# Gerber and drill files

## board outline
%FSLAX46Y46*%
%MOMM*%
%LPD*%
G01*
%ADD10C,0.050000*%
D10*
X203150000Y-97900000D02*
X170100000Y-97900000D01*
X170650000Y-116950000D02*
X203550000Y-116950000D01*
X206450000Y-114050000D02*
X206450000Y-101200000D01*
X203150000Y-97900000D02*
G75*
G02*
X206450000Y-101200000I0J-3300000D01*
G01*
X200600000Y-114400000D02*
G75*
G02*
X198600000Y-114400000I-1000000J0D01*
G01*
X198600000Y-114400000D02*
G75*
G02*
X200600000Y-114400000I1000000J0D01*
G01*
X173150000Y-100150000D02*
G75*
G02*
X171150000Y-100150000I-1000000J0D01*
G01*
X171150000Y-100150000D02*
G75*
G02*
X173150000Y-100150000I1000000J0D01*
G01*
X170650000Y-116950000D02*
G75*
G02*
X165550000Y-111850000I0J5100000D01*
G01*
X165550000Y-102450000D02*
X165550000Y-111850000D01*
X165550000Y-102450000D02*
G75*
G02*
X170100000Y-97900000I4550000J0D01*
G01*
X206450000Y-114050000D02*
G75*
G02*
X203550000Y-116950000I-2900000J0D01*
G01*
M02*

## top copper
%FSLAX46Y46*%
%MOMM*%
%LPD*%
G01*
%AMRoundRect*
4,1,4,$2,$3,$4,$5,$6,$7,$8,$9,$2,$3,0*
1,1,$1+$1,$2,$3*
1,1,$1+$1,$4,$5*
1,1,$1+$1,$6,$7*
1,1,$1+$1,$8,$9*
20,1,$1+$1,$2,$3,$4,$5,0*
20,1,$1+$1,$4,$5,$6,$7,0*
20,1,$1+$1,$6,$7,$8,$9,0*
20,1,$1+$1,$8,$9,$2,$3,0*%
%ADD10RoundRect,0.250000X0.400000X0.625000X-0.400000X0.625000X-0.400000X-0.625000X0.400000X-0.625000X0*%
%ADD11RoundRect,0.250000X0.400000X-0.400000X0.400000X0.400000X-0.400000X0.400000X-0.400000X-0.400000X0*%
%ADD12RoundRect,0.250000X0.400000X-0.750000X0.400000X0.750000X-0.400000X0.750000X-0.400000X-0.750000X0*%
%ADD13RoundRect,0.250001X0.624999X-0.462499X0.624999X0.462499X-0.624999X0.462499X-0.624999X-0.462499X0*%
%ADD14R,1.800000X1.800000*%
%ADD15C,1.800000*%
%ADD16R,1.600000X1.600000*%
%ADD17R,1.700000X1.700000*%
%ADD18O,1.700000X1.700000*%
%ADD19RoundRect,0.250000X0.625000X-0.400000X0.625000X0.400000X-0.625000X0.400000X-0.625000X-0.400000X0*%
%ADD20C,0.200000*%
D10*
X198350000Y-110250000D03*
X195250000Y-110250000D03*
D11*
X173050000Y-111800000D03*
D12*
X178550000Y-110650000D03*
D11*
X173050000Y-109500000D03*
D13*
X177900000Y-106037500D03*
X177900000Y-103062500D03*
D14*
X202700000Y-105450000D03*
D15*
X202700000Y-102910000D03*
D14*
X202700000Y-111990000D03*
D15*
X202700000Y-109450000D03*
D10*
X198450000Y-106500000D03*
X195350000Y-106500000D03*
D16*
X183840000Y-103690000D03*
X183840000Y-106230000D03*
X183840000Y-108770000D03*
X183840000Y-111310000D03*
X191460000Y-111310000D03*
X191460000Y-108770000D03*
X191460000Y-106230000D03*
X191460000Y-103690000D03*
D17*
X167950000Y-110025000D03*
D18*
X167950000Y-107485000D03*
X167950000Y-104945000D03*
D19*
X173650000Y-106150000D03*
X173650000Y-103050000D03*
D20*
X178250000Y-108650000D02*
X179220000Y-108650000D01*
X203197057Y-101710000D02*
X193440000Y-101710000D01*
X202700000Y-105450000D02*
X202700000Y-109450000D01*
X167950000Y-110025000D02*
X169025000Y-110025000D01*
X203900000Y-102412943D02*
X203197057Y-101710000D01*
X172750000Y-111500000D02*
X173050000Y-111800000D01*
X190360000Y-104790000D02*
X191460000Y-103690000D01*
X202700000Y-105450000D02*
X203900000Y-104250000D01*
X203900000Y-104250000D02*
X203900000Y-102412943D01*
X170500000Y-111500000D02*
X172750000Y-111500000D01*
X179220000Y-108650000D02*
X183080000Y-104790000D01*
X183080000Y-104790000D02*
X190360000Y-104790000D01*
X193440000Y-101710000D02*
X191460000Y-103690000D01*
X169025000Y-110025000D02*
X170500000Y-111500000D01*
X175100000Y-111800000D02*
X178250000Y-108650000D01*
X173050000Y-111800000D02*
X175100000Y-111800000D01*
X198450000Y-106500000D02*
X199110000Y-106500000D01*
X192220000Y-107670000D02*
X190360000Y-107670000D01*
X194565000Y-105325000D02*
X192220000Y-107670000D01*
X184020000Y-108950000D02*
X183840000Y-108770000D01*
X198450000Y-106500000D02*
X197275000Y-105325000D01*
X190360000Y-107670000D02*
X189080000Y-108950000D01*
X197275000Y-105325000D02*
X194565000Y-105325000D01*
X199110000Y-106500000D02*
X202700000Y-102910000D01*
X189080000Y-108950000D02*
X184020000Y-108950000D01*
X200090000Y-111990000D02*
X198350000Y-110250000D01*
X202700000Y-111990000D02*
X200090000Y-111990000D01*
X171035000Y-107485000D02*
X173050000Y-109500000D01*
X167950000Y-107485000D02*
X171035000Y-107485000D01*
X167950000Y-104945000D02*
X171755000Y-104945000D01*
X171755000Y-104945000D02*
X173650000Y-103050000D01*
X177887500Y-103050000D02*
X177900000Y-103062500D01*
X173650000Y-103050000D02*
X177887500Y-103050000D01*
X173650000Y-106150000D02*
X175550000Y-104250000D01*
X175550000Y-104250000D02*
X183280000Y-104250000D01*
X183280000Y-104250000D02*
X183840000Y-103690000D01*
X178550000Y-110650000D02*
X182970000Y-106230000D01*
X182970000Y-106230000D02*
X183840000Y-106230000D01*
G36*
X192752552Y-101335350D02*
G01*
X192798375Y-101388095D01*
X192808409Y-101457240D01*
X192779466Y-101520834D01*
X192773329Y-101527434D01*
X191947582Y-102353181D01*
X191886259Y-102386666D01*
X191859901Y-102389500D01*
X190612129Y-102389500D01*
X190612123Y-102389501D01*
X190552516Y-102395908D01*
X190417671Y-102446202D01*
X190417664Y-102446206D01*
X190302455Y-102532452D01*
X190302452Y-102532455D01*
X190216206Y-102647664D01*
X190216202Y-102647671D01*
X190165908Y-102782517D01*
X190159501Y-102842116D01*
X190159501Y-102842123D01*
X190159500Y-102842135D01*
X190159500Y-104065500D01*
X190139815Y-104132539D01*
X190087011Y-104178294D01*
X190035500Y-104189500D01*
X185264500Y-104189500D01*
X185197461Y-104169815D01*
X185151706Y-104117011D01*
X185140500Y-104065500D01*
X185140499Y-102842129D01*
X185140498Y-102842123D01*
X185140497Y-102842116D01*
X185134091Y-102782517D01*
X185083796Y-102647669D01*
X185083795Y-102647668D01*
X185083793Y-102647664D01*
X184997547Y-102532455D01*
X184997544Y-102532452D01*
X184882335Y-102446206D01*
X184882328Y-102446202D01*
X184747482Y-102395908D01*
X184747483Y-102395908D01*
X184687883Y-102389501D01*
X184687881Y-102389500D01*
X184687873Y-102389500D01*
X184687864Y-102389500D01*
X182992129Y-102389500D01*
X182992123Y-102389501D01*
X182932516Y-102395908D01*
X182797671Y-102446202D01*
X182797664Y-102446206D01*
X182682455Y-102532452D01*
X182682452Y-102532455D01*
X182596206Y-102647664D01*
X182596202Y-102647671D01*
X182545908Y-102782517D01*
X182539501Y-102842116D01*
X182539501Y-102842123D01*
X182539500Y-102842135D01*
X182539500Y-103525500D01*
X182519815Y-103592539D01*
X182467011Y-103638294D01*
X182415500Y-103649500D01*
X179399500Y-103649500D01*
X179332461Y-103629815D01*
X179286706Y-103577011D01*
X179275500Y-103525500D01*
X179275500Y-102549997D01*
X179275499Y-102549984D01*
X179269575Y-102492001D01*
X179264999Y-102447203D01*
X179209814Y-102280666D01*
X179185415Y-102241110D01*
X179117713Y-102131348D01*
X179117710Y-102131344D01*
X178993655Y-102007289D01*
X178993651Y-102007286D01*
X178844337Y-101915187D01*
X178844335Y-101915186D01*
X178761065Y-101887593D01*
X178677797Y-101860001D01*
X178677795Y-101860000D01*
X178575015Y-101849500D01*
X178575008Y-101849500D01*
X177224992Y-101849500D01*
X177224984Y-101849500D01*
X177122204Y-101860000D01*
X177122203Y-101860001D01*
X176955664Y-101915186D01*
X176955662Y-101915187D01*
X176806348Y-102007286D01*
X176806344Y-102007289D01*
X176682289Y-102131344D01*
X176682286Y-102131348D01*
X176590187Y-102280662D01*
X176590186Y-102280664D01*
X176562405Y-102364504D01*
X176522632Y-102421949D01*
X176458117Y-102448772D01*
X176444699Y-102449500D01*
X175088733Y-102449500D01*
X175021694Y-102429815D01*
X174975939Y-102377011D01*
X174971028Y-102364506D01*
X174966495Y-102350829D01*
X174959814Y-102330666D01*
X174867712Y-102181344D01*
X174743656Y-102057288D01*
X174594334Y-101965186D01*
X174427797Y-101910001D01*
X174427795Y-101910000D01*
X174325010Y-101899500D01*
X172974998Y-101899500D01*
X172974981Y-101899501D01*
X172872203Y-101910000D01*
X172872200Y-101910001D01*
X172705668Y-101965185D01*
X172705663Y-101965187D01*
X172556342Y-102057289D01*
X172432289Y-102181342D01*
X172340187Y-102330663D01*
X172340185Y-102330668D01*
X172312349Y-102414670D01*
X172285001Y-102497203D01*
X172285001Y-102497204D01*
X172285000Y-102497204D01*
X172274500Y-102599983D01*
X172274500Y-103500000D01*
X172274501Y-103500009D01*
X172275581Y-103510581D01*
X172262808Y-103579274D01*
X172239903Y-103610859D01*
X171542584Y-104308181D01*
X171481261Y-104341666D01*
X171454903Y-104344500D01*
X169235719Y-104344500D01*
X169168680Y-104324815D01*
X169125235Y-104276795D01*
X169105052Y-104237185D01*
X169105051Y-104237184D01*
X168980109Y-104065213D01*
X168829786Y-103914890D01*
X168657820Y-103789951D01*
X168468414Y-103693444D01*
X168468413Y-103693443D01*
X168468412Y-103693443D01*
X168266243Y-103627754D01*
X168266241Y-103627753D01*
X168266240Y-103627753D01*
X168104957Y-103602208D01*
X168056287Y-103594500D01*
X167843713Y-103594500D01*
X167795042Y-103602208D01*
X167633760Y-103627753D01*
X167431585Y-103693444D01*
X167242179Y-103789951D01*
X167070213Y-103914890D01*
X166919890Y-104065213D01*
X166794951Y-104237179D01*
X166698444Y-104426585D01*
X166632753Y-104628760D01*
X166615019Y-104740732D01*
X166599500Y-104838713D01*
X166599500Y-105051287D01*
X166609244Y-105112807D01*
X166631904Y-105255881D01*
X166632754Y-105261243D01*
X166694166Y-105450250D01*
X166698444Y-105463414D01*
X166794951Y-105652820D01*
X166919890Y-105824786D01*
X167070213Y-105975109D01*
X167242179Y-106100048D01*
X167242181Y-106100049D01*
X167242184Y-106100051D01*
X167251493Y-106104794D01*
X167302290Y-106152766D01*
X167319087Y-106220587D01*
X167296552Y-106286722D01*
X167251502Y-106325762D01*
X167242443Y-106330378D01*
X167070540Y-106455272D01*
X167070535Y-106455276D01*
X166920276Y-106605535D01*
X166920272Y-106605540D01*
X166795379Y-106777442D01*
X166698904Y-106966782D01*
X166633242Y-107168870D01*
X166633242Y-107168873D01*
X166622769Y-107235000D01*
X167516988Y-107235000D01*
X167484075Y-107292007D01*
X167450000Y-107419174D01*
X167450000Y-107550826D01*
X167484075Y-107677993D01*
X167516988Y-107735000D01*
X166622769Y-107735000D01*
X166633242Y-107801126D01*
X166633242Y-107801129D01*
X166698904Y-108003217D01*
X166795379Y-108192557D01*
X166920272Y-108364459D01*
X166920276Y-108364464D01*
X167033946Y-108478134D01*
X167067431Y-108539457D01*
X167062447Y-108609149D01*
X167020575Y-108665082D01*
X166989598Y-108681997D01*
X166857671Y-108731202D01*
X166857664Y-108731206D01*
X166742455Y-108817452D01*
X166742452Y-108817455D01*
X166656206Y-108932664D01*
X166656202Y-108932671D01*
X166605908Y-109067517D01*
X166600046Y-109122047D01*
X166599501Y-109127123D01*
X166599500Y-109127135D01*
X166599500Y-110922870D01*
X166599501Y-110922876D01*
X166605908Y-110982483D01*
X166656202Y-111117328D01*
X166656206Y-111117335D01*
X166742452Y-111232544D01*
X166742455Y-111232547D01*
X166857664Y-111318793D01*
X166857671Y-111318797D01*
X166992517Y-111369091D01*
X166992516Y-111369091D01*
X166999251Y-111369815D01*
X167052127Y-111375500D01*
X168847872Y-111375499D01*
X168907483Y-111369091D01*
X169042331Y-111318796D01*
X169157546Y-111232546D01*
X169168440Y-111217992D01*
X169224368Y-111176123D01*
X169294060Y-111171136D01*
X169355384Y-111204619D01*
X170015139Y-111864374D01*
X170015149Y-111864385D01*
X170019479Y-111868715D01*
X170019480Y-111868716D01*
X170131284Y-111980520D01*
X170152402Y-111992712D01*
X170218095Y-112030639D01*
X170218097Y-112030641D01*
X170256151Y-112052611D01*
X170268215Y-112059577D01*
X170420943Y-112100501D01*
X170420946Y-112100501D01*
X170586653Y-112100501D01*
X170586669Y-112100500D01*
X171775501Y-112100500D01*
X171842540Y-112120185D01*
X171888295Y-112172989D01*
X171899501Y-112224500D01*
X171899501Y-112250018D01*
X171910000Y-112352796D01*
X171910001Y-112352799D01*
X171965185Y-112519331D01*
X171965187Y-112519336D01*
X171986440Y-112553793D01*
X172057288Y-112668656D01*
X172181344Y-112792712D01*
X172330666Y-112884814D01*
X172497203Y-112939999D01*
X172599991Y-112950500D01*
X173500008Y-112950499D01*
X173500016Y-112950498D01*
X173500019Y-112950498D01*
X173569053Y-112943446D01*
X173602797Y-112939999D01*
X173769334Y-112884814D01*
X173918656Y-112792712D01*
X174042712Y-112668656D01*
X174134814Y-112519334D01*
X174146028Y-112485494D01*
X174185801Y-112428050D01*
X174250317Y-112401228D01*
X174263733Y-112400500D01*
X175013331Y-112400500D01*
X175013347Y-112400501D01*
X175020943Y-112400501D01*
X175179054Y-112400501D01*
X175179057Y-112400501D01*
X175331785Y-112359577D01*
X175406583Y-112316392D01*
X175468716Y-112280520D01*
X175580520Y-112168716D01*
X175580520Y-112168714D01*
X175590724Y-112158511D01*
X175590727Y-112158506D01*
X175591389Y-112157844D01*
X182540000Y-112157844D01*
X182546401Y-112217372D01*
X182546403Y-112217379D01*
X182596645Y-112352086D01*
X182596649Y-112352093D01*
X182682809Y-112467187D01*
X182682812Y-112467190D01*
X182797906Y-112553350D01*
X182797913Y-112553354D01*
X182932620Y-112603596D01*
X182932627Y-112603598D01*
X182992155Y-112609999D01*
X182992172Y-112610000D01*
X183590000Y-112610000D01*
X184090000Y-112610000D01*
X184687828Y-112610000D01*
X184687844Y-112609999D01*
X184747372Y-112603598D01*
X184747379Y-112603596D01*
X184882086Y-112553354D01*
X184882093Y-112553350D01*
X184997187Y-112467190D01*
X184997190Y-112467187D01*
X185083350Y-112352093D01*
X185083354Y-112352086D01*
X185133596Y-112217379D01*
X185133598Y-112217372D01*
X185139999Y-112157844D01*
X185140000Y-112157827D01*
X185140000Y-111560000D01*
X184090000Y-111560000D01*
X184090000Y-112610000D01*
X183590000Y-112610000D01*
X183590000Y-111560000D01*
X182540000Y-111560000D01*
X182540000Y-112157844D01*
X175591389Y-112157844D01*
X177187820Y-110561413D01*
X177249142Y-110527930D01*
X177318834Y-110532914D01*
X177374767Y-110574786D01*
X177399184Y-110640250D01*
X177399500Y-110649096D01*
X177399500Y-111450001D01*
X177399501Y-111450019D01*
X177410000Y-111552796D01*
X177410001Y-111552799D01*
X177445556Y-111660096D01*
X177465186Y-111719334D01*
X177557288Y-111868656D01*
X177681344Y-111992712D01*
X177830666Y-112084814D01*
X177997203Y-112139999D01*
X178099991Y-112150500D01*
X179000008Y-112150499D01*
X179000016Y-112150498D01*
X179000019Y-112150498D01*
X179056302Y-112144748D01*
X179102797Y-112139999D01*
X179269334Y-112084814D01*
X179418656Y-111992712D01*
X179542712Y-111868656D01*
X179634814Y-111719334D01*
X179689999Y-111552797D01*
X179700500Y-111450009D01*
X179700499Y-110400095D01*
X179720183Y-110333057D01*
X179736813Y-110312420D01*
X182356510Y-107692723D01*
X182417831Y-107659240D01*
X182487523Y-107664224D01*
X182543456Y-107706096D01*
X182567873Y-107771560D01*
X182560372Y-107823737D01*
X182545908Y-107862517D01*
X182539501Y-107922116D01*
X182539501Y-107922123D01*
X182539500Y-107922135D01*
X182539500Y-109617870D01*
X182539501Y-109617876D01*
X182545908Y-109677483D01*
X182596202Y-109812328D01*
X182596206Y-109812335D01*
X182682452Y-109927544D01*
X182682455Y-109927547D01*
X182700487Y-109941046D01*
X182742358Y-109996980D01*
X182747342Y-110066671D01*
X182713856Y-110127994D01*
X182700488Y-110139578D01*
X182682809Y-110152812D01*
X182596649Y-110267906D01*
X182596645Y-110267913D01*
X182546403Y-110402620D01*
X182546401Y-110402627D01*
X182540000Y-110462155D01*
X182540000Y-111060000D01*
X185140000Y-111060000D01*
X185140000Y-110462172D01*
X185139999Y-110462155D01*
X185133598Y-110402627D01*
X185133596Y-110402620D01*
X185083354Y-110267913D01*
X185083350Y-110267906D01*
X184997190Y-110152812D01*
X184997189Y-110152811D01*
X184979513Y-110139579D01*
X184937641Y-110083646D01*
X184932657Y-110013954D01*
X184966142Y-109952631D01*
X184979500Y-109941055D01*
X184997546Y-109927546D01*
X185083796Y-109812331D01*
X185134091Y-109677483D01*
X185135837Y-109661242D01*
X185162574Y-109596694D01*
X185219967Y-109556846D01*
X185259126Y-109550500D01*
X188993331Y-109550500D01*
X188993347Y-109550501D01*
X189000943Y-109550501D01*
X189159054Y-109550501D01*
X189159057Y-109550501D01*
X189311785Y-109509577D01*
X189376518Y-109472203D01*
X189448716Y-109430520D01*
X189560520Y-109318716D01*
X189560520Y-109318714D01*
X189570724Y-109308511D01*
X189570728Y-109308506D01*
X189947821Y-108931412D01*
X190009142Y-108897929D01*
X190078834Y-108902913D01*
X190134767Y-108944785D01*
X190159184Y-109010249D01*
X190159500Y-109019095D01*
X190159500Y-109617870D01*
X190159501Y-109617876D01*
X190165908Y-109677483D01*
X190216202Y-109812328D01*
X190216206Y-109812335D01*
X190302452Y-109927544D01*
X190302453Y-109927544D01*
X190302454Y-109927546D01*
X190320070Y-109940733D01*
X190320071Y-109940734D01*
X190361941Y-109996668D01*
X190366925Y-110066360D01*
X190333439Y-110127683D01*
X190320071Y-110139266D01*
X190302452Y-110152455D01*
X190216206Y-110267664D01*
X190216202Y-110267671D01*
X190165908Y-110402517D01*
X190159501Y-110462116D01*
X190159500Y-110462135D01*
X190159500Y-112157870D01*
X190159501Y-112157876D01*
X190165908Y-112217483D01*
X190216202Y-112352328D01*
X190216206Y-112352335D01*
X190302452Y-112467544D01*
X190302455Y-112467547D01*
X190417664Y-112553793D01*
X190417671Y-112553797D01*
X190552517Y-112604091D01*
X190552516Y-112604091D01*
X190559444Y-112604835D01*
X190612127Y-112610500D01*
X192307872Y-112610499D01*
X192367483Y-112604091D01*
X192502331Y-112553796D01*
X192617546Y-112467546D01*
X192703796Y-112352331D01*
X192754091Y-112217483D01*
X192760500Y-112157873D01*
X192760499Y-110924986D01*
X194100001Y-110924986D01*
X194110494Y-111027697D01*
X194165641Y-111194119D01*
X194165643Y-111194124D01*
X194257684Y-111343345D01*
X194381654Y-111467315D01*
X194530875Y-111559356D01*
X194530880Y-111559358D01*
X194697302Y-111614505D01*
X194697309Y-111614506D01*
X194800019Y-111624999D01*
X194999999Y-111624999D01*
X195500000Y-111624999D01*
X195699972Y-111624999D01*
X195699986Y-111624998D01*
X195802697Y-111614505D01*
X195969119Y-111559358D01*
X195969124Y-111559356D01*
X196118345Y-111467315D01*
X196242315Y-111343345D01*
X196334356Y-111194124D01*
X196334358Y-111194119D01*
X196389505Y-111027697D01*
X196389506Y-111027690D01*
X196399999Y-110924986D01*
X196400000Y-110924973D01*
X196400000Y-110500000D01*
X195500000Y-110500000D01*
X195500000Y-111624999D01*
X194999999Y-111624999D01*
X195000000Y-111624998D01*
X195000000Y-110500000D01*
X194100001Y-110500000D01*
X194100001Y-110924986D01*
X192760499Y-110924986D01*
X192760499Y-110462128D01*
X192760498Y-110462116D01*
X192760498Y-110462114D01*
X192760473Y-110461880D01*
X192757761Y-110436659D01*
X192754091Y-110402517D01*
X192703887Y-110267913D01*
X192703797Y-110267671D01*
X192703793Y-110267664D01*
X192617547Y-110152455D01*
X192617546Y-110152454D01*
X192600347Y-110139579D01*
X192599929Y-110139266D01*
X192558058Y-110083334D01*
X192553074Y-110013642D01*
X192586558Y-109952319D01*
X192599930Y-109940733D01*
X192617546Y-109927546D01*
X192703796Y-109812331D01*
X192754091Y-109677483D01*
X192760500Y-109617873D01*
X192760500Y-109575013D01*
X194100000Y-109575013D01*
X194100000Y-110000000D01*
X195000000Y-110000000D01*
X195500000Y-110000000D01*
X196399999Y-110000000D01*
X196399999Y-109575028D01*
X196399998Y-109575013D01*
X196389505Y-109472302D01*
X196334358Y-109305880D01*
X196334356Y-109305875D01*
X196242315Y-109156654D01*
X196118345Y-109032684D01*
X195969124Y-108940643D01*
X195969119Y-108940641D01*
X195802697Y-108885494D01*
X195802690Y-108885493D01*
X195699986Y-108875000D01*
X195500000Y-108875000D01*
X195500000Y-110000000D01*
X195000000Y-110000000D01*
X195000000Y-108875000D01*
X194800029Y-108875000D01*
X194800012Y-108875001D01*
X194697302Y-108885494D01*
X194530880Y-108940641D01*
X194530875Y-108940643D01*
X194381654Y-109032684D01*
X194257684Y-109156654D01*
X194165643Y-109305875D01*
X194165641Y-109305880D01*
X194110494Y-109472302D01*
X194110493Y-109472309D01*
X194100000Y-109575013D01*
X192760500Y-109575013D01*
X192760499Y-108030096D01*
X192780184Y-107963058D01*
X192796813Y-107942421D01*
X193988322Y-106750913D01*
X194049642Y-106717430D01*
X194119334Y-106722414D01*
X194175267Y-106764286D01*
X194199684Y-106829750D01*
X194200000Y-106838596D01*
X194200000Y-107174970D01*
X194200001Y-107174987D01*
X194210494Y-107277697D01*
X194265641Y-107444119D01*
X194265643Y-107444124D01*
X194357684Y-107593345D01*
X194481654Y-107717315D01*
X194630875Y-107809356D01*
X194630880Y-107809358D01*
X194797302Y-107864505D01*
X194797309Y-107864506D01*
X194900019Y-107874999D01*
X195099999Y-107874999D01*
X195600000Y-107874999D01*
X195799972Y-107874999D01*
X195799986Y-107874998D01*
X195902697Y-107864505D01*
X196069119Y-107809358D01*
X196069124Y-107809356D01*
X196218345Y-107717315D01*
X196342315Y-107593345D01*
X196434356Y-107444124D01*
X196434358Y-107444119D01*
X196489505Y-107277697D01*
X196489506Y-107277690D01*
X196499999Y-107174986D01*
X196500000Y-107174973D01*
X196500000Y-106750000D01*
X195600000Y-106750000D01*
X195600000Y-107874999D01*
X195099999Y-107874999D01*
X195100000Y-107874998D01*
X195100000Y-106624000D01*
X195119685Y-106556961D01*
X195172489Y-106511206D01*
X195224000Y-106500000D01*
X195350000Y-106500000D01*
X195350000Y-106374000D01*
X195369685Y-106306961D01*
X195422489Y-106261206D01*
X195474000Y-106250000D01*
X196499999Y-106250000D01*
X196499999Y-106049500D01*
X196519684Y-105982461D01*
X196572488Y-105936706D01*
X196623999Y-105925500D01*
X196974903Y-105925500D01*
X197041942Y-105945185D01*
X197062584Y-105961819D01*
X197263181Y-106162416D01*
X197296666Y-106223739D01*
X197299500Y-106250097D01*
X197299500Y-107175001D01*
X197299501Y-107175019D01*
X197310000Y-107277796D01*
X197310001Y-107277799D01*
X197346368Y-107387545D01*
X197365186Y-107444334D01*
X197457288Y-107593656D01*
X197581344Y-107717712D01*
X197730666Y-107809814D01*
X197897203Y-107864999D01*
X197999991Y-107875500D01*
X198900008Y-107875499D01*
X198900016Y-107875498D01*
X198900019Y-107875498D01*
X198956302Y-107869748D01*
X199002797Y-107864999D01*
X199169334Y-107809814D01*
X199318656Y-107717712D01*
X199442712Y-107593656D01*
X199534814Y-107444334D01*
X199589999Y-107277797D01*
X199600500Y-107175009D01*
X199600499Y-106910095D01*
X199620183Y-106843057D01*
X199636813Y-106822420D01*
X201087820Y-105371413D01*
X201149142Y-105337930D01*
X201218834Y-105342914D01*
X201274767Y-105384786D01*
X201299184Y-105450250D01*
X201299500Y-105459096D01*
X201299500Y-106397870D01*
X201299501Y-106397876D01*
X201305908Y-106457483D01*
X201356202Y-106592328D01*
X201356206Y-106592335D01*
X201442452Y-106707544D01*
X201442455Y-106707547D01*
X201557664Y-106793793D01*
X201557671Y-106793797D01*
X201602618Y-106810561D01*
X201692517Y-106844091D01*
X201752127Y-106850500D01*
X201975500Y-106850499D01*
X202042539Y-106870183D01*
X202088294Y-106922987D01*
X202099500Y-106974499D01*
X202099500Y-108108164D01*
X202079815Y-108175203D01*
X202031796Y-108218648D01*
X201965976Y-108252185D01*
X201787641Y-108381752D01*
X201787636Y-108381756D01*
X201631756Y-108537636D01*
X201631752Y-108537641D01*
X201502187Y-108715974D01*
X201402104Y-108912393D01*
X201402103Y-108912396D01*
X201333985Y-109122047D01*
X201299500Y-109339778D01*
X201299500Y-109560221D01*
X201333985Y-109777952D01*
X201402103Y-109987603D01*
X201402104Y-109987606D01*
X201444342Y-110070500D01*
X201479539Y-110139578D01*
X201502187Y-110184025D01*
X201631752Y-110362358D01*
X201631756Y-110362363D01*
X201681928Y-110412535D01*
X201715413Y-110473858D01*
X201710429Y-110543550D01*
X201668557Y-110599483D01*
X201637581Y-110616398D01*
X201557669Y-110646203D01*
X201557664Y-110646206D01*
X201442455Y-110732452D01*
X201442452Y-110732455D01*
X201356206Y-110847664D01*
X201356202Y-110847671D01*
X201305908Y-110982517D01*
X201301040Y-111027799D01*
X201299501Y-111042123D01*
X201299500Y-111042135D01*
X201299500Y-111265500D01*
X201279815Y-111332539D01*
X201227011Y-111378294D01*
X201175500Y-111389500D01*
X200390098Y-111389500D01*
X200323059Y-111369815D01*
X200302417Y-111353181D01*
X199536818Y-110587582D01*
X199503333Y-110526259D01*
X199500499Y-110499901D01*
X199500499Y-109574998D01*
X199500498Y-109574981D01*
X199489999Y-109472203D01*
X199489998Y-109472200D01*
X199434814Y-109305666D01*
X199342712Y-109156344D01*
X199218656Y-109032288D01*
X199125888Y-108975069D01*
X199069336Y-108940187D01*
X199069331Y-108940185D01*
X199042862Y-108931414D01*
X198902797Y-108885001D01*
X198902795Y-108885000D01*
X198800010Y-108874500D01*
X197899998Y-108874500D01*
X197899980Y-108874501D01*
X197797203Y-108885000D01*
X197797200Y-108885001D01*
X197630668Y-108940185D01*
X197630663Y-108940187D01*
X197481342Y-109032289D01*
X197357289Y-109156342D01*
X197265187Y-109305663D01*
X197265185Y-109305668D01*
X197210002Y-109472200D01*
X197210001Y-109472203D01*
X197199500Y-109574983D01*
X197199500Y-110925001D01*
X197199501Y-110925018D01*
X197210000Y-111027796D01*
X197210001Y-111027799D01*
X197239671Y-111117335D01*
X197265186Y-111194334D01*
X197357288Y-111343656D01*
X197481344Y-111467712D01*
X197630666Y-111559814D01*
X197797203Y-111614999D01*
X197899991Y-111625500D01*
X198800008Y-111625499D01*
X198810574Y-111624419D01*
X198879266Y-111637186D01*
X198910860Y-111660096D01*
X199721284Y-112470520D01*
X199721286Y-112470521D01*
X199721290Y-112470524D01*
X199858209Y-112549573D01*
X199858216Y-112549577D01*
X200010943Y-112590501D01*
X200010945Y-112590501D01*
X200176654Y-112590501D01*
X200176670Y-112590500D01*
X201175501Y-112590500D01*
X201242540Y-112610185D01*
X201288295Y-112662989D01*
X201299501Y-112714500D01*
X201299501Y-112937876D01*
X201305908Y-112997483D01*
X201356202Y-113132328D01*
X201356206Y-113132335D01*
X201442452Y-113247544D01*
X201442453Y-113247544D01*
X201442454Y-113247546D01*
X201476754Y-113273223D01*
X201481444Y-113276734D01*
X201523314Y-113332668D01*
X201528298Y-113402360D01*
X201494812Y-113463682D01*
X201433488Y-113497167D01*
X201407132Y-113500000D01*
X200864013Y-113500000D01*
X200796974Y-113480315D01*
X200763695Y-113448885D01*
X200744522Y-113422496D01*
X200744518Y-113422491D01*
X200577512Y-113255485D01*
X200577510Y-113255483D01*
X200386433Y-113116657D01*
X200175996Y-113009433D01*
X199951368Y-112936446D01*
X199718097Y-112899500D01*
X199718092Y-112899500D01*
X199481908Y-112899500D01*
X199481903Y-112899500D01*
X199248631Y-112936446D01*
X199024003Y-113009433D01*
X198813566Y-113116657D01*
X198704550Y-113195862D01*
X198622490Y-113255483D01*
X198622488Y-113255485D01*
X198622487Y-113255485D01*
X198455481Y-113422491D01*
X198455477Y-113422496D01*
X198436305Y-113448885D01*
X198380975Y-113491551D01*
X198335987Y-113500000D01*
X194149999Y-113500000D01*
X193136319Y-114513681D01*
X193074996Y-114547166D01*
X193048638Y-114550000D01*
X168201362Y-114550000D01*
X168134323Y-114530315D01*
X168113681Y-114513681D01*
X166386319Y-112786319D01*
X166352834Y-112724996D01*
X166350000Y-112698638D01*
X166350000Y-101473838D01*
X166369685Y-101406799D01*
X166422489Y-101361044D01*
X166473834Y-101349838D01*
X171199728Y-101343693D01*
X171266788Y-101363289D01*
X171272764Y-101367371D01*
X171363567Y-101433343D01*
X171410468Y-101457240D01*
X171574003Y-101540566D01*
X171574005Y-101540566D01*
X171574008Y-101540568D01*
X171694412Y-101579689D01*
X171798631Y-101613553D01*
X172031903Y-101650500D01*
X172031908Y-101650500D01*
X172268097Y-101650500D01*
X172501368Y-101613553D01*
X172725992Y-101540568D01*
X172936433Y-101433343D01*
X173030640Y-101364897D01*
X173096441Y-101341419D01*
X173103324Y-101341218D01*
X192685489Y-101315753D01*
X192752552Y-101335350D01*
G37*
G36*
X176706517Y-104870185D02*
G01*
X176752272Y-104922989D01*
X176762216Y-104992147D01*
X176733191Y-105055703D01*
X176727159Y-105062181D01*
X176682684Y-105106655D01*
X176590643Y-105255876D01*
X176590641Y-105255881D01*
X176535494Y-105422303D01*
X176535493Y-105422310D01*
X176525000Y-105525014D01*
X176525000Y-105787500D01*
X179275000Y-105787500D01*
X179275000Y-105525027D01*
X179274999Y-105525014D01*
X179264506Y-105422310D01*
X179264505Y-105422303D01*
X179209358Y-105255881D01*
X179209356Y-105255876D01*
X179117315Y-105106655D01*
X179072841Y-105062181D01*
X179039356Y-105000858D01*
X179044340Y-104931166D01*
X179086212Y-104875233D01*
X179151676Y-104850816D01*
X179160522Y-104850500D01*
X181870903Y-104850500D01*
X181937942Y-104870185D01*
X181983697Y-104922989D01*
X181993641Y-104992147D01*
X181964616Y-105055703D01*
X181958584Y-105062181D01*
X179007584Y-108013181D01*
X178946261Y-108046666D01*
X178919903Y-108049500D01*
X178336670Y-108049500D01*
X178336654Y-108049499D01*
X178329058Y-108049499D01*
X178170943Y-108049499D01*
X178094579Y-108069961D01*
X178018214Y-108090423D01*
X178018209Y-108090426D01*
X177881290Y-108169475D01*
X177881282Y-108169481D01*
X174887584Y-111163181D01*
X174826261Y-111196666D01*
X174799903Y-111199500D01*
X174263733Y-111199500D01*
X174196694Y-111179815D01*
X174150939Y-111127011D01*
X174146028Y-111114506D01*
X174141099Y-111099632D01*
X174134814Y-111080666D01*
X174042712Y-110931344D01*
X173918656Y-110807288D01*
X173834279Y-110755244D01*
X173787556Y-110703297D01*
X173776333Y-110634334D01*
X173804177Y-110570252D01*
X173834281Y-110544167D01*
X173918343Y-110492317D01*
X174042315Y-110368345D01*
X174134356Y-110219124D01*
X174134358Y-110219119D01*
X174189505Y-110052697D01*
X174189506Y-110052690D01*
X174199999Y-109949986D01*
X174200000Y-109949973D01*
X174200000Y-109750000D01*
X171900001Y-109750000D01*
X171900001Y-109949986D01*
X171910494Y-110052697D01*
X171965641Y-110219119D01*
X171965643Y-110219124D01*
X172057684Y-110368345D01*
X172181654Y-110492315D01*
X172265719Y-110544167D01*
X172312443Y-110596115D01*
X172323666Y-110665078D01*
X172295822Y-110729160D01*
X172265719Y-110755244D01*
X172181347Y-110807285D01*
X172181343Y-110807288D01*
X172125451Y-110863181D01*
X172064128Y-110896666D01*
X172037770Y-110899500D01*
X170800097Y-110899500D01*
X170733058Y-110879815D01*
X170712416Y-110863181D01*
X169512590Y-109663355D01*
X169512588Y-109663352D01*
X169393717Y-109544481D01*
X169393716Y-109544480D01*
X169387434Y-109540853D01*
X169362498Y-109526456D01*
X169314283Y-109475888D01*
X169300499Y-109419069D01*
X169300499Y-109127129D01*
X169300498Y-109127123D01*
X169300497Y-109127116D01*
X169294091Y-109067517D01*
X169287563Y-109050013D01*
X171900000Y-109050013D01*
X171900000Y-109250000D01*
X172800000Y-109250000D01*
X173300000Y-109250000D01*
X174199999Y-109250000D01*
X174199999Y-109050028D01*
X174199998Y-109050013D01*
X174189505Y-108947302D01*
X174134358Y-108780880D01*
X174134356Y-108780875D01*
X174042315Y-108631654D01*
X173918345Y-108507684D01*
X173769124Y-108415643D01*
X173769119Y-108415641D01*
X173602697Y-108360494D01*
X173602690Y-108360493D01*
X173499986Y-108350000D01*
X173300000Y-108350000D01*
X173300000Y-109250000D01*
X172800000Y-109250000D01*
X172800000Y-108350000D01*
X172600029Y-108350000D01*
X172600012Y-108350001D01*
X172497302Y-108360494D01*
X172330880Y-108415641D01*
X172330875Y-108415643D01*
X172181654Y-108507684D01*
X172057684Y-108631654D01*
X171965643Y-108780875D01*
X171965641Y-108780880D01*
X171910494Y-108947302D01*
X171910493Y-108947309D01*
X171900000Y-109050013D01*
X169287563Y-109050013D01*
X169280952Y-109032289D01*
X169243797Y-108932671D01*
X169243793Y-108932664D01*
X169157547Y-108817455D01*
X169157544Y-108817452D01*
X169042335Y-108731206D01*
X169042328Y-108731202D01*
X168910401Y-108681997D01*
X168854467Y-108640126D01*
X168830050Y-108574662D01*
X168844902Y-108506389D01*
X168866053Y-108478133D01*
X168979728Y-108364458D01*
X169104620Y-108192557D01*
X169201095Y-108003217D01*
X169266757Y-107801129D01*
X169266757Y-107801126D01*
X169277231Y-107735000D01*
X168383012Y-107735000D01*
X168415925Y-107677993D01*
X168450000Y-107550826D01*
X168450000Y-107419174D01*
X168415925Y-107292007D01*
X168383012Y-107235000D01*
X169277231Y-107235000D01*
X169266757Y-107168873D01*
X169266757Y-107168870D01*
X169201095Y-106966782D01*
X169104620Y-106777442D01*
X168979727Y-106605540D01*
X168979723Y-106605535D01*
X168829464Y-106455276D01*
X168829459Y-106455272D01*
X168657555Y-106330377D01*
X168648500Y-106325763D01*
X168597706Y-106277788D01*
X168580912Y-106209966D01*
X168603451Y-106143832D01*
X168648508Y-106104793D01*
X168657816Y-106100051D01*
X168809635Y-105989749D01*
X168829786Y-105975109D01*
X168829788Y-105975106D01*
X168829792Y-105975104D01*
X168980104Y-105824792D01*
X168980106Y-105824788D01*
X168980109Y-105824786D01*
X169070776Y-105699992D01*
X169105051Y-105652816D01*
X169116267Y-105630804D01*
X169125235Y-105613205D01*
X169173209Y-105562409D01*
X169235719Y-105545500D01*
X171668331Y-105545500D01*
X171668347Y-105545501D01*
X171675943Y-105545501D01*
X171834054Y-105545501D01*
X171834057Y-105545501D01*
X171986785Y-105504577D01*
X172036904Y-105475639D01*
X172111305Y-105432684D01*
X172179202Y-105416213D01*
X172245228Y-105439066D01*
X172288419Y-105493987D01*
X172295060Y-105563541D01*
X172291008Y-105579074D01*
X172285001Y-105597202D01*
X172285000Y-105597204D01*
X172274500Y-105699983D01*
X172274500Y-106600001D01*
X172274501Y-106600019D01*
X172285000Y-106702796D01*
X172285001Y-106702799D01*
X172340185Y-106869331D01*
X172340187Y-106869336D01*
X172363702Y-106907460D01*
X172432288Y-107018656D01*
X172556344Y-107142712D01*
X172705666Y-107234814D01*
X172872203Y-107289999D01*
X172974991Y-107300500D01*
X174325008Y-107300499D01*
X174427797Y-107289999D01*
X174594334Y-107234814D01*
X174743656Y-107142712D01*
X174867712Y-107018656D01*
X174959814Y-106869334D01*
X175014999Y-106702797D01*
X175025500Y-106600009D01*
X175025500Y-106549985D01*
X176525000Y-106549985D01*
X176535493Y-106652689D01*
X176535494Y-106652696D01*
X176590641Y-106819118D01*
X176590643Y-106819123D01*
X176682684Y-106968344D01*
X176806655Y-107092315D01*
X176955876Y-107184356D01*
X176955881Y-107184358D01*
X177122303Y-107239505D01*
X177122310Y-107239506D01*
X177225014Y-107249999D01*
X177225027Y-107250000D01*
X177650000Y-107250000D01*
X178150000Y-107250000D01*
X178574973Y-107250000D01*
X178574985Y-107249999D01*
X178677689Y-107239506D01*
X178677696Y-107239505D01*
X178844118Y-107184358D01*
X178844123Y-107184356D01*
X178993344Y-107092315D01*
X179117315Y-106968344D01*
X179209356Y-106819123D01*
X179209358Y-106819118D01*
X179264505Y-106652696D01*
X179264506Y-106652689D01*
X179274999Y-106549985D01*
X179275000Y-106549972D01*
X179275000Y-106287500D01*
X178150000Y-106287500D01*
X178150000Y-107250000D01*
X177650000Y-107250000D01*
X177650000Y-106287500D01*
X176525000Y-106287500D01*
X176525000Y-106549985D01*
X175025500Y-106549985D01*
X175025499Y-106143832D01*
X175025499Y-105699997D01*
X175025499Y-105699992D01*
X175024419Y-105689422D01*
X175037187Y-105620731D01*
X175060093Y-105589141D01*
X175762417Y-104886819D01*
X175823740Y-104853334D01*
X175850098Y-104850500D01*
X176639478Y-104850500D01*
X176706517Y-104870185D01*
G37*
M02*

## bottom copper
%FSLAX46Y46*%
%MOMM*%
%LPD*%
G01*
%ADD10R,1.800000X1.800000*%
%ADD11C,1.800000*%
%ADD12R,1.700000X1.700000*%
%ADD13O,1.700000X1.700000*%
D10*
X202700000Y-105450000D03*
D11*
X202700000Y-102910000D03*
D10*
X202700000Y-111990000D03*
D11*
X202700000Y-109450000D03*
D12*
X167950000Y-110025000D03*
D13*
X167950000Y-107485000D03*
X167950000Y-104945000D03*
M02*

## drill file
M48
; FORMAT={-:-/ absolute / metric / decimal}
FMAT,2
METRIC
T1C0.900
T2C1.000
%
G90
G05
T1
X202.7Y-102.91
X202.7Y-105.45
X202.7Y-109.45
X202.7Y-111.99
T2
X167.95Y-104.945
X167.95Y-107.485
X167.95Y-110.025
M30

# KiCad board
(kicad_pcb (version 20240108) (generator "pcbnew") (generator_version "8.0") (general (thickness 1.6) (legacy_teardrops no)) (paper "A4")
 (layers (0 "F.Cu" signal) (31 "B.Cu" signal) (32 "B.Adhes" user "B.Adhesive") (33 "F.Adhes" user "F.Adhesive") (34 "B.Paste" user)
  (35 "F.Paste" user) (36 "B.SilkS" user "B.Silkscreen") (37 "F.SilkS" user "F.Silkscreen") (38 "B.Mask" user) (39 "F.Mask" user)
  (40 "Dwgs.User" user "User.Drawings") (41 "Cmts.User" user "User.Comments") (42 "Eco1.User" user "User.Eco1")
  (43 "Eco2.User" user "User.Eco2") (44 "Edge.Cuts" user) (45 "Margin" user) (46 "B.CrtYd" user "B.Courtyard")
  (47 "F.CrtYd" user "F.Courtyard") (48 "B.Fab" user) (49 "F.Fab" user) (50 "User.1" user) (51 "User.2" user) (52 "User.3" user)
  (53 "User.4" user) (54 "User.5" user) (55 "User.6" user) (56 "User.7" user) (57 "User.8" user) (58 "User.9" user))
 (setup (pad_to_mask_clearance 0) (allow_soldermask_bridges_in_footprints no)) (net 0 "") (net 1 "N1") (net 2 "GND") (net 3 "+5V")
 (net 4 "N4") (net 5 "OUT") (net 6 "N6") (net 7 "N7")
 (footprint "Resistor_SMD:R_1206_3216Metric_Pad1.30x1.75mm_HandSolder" (layer "F.Cu") (at 196.8 110.25 180)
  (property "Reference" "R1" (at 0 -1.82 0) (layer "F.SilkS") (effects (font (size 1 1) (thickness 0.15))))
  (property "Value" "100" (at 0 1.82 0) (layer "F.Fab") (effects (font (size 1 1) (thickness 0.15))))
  (pad "1" smd roundrect (at -1.55 0 180) (size 1.3 1.75) (layers "F.Cu" "F.Paste" "F.Mask") (roundrect_rratio 0.192308) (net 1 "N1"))
  (pad "2" smd roundrect (at 1.55 0 180) (size 1.3 1.75) (layers "F.Cu" "F.Paste" "F.Mask") (roundrect_rratio 0.192308) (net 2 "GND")))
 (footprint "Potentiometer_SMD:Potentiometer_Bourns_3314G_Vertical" (layer "F.Cu") (at 175.8 110.65 90)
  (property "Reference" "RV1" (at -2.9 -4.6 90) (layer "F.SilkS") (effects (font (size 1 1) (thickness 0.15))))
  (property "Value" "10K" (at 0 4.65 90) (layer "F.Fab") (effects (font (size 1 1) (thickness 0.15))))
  (pad "1" smd roundrect (at -1.15 -2.75 90) (size 1.3 1.3) (layers "F.Cu" "F.Paste" "F.Mask") (roundrect_rratio 0.1923076923) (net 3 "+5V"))
  (pad "2" smd roundrect (at 0 2.75 90) (size 2 1.3) (layers "F.Cu" "F.Paste" "F.Mask") (roundrect_rratio 0.1923076923) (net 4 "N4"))
  (pad "3" smd roundrect (at 1.15 -2.75 90) (size 1.3 1.3) (layers "F.Cu" "F.Paste" "F.Mask") (roundrect_rratio 0.1923076923) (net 2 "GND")))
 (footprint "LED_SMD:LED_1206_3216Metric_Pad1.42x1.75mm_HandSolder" (layer "F.Cu") (at 177.9 104.55 90)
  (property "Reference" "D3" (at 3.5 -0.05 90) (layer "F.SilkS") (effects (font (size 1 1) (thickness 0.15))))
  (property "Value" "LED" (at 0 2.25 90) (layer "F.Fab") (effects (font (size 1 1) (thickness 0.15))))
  (pad "1" smd roundrect (at -1.4875 0 90) (size 1.425 1.75) (layers "F.Cu" "F.Paste" "F.Mask") (roundrect_rratio 0.175439) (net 2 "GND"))
  (pad "2" smd roundrect (at 1.4875 0 90) (size 1.425 1.75) (layers "F.Cu" "F.Paste" "F.Mask") (roundrect_rratio 0.175439) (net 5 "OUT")))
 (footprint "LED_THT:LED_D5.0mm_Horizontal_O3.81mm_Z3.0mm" (layer "F.Cu") (at 202.7 105.45 90)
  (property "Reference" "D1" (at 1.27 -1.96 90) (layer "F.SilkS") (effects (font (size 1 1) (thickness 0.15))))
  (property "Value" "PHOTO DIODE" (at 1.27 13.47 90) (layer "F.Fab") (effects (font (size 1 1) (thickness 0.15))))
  (pad "1" thru_hole rect (at 0 0 90) (size 1.8 1.8) (drill 0.9) (layers "*.Cu" "*.Mask") (remove_unused_layers no) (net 3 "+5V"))
  (pad "2" thru_hole circle (at 2.54 0 90) (size 1.8 1.8) (drill 0.9) (layers "*.Cu" "*.Mask") (remove_unused_layers no) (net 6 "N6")))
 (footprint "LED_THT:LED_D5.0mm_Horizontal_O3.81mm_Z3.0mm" (layer "F.Cu") (at 202.7 111.99 90)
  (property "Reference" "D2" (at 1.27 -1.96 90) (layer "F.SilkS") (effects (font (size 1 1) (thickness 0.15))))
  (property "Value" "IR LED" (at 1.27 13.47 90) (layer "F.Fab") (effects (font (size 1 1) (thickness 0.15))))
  (pad "1" thru_hole rect (at 0 0 90) (size 1.8 1.8) (drill 0.9) (layers "*.Cu" "*.Mask") (remove_unused_layers no) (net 1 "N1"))
  (pad "2" thru_hole circle (at 2.54 0 90) (size 1.8 1.8) (drill 0.9) (layers "*.Cu" "*.Mask") (remove_unused_layers no) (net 3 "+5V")))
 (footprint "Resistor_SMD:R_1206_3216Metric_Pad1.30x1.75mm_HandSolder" (layer "F.Cu") (at 196.9 106.5 180)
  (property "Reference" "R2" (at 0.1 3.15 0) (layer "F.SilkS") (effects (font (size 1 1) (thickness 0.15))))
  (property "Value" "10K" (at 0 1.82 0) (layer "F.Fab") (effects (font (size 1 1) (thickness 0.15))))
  (pad "1" smd roundrect (at -1.55 0 180) (size 1.3 1.75) (layers "F.Cu" "F.Paste" "F.Mask") (roundrect_rratio 0.192308) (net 6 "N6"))
  (pad "2" smd roundrect (at 1.55 0 180) (size 1.3 1.75) (layers "F.Cu" "F.Paste" "F.Mask") (roundrect_rratio 0.192308) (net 2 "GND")))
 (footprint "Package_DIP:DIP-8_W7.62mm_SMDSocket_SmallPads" (layer "F.Cu") (at 187.65 107.5)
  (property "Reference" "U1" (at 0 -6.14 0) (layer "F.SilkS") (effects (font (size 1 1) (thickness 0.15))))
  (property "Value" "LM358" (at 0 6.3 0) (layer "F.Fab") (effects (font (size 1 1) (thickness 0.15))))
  (pad "1" smd rect (at -3.81 -3.81) (size 1.6 1.6) (layers "F.Cu" "F.Paste" "F.Mask") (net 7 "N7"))
  (pad "2" smd rect (at -3.81 -1.27) (size 1.6 1.6) (layers "F.Cu" "F.Paste" "F.Mask") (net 4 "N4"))
  (pad "3" smd rect (at -3.81 1.27) (size 1.6 1.6) (layers "F.Cu" "F.Paste" "F.Mask") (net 6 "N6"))
  (pad "4" smd rect (at -3.81 3.81) (size 1.6 1.6) (layers "F.Cu" "F.Paste" "F.Mask") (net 2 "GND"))
  (pad "5" smd rect (at 3.81 3.81) (size 1.6 1.6) (layers "F.Cu" "F.Paste" "F.Mask"))
  (pad "6" smd rect (at 3.81 1.27) (size 1.6 1.6) (layers "F.Cu" "F.Paste" "F.Mask"))
  (pad "7" smd rect (at 3.81 -1.27) (size 1.6 1.6) (layers "F.Cu" "F.Paste" "F.Mask"))
  (pad "8" smd rect (at 3.81 -3.81) (size 1.6 1.6) (layers "F.Cu" "F.Paste" "F.Mask") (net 3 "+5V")))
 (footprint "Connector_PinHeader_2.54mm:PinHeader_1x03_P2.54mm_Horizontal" (layer "F.Cu") (at 167.95 110.025 180)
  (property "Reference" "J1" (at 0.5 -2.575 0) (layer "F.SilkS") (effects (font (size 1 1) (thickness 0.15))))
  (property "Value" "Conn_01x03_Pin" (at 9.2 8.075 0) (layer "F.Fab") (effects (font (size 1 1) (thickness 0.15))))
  (pad "1" thru_hole rect (at 0 0 180) (size 1.7 1.7) (drill 1) (layers "*.Cu" "*.Mask") (remove_unused_layers no) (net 3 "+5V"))
  (pad "2" thru_hole oval (at 0 2.54 180) (size 1.7 1.7) (drill 1) (layers "*.Cu" "*.Mask") (remove_unused_layers no) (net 2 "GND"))
  (pad "3" thru_hole oval (at 0 5.08 180) (size 1.7 1.7) (drill 1) (layers "*.Cu" "*.Mask") (remove_unused_layers no) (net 5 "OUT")))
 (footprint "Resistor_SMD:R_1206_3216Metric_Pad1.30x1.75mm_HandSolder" (layer "F.Cu") (at 173.65 104.6 90)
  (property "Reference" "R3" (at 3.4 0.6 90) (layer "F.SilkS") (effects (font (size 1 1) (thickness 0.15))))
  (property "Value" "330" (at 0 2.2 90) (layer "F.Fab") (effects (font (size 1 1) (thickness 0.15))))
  (pad "1" smd roundrect (at -1.55 0 90) (size 1.3 1.75) (layers "F.Cu" "F.Paste" "F.Mask") (roundrect_rratio 0.192308) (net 7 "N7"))
  (pad "2" smd roundrect (at 1.55 0 90) (size 1.3 1.75) (layers "F.Cu" "F.Paste" "F.Mask") (roundrect_rratio 0.192308) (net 5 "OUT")))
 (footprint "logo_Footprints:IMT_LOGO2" (layer "B.Cu") (at 187.825 102.12 180)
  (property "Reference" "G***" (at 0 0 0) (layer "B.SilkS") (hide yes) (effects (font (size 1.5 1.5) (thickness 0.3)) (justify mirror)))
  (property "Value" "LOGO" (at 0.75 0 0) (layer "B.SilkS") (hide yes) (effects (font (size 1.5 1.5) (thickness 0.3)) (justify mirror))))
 (gr_line (start 203.15 97.9) (end 170.1 97.9) (stroke (width 0.05) (type default)) (layer "Edge.Cuts"))
 (gr_line (start 170.65 116.95) (end 203.55 116.95) (stroke (width 0.05) (type default)) (layer "Edge.Cuts"))
 (gr_line (start 206.45 114.05) (end 206.45 101.2) (stroke (width 0.05) (type default)) (layer "Edge.Cuts"))
 (gr_arc (start 203.15 97.9) (mid 205.483452 98.866548) (end 206.45 101.2) (stroke (width 0.05) (type default)) (layer "Edge.Cuts"))
 (gr_circle (center 199.6 114.4) (end 199.6 113.4) (stroke (width 0.05) (type default)) (fill none) (layer "Edge.Cuts"))
 (gr_circle (center 172.15 100.15) (end 172.15 99.15) (stroke (width 0.05) (type default)) (fill none) (layer "Edge.Cuts"))
 (gr_arc (start 170.65 116.95) (mid 167.043755 115.456245) (end 165.55 111.85) (stroke (width 0.05) (type default)) (layer "Edge.Cuts"))
 (gr_line (start 165.55 102.45) (end 165.55 111.85) (stroke (width 0.05) (type default)) (layer "Edge.Cuts"))
 (gr_arc (start 165.55 102.45) (mid 166.882664 99.232664) (end 170.1 97.9) (stroke (width 0.05) (type default)) (layer "Edge.Cuts"))
 (gr_arc (start 206.45 114.05) (mid 205.60061 116.10061) (end 203.55 116.95) (stroke (width 0.05) (type default)) (layer "Edge.Cuts"))
 (segment (start 178.25 108.65) (end 179.22 108.65) (width 0.2) (layer "F.Cu") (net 3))
 (segment (start 203.197057 101.71) (end 193.44 101.71) (width 0.2) (layer "F.Cu") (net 3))
 (segment (start 202.7 105.45) (end 202.7 109.45) (width 0.2) (layer "F.Cu") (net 3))
 (segment (start 167.95 110.025) (end 169.025 110.025) (width 0.2) (layer "F.Cu") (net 3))
 (segment (start 203.9 102.412943) (end 203.197057 101.71) (width 0.2) (layer "F.Cu") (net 3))
 (segment (start 172.75 111.5) (end 173.05 111.8) (width 0.2) (layer "F.Cu") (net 3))
 (segment (start 190.36 104.79) (end 191.46 103.69) (width 0.2) (layer "F.Cu") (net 3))
 (segment (start 202.7 105.45) (end 203.9 104.25) (width 0.2) (layer "F.Cu") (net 3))
 (segment (start 203.9 104.25) (end 203.9 102.412943) (width 0.2) (layer "F.Cu") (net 3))
 (segment (start 170.5 111.5) (end 172.75 111.5) (width 0.2) (layer "F.Cu") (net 3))
 (segment (start 179.22 108.65) (end 183.08 104.79) (width 0.2) (layer "F.Cu") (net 3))
 (segment (start 183.08 104.79) (end 190.36 104.79) (width 0.2) (layer "F.Cu") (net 3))
 (segment (start 193.44 101.71) (end 191.46 103.69) (width 0.2) (layer "F.Cu") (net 3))
 (segment (start 169.025 110.025) (end 170.5 111.5) (width 0.2) (layer "F.Cu") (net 3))
 (segment (start 175.1 111.8) (end 178.25 108.65) (width 0.2) (layer "F.Cu") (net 3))
 (segment (start 173.05 111.8) (end 175.1 111.8) (width 0.2) (layer "F.Cu") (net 3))
 (segment (start 198.45 106.5) (end 199.11 106.5) (width 0.2) (layer "F.Cu") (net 6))
 (segment (start 192.22 107.67) (end 190.36 107.67) (width 0.2) (layer "F.Cu") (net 6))
 (segment (start 194.565 105.325) (end 192.22 107.67) (width 0.2) (layer "F.Cu") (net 6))
 (segment (start 184.02 108.95) (end 183.84 108.77) (width 0.2) (layer "F.Cu") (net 6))
 (segment (start 198.45 106.5) (end 197.275 105.325) (width 0.2) (layer "F.Cu") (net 6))
 (segment (start 190.36 107.67) (end 189.08 108.95) (width 0.2) (layer "F.Cu") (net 6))
 (segment (start 197.275 105.325) (end 194.565 105.325) (width 0.2) (layer "F.Cu") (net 6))
 (segment (start 199.11 106.5) (end 202.7 102.91) (width 0.2) (layer "F.Cu") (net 6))
 (segment (start 189.08 108.95) (end 184.02 108.95) (width 0.2) (layer "F.Cu") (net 6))
 (segment (start 200.09 111.99) (end 198.35 110.25) (width 0.2) (layer "F.Cu") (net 1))
 (segment (start 202.7 111.99) (end 200.09 111.99) (width 0.2) (layer "F.Cu") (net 1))
 (segment (start 171.035 107.485) (end 173.05 109.5) (width 0.2) (layer "F.Cu") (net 2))
 (segment (start 167.95 107.485) (end 171.035 107.485) (width 0.2) (layer "F.Cu") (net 2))
 (segment (start 167.95 104.945) (end 171.755 104.945) (width 0.2) (layer "F.Cu") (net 5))
 (segment (start 171.755 104.945) (end 173.65 103.05) (width 0.2) (layer "F.Cu") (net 5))
 (segment (start 177.8875 103.05) (end 177.9 103.0625) (width 0.2) (layer "F.Cu") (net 5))
 (segment (start 173.65 103.05) (end 177.8875 103.05) (width 0.2) (layer "F.Cu") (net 5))
 (segment (start 173.65 106.15) (end 175.55 104.25) (width 0.2) (layer "F.Cu") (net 7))
 (segment (start 175.55 104.25) (end 183.28 104.25) (width 0.2) (layer "F.Cu") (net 7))
 (segment (start 183.28 104.25) (end 183.84 103.69) (width 0.2) (layer "F.Cu") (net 7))
 (segment (start 178.55 110.65) (end 182.97 106.23) (width 0.2) (layer "F.Cu") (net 4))
 (segment (start 182.97 106.23) (end 183.84 106.23) (width 0.2) (layer "F.Cu") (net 4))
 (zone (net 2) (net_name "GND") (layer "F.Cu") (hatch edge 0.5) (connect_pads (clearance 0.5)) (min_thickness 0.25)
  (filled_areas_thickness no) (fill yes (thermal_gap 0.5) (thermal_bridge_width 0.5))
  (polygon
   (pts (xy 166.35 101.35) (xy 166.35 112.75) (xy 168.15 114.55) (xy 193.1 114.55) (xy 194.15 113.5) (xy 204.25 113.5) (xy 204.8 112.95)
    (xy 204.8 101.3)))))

